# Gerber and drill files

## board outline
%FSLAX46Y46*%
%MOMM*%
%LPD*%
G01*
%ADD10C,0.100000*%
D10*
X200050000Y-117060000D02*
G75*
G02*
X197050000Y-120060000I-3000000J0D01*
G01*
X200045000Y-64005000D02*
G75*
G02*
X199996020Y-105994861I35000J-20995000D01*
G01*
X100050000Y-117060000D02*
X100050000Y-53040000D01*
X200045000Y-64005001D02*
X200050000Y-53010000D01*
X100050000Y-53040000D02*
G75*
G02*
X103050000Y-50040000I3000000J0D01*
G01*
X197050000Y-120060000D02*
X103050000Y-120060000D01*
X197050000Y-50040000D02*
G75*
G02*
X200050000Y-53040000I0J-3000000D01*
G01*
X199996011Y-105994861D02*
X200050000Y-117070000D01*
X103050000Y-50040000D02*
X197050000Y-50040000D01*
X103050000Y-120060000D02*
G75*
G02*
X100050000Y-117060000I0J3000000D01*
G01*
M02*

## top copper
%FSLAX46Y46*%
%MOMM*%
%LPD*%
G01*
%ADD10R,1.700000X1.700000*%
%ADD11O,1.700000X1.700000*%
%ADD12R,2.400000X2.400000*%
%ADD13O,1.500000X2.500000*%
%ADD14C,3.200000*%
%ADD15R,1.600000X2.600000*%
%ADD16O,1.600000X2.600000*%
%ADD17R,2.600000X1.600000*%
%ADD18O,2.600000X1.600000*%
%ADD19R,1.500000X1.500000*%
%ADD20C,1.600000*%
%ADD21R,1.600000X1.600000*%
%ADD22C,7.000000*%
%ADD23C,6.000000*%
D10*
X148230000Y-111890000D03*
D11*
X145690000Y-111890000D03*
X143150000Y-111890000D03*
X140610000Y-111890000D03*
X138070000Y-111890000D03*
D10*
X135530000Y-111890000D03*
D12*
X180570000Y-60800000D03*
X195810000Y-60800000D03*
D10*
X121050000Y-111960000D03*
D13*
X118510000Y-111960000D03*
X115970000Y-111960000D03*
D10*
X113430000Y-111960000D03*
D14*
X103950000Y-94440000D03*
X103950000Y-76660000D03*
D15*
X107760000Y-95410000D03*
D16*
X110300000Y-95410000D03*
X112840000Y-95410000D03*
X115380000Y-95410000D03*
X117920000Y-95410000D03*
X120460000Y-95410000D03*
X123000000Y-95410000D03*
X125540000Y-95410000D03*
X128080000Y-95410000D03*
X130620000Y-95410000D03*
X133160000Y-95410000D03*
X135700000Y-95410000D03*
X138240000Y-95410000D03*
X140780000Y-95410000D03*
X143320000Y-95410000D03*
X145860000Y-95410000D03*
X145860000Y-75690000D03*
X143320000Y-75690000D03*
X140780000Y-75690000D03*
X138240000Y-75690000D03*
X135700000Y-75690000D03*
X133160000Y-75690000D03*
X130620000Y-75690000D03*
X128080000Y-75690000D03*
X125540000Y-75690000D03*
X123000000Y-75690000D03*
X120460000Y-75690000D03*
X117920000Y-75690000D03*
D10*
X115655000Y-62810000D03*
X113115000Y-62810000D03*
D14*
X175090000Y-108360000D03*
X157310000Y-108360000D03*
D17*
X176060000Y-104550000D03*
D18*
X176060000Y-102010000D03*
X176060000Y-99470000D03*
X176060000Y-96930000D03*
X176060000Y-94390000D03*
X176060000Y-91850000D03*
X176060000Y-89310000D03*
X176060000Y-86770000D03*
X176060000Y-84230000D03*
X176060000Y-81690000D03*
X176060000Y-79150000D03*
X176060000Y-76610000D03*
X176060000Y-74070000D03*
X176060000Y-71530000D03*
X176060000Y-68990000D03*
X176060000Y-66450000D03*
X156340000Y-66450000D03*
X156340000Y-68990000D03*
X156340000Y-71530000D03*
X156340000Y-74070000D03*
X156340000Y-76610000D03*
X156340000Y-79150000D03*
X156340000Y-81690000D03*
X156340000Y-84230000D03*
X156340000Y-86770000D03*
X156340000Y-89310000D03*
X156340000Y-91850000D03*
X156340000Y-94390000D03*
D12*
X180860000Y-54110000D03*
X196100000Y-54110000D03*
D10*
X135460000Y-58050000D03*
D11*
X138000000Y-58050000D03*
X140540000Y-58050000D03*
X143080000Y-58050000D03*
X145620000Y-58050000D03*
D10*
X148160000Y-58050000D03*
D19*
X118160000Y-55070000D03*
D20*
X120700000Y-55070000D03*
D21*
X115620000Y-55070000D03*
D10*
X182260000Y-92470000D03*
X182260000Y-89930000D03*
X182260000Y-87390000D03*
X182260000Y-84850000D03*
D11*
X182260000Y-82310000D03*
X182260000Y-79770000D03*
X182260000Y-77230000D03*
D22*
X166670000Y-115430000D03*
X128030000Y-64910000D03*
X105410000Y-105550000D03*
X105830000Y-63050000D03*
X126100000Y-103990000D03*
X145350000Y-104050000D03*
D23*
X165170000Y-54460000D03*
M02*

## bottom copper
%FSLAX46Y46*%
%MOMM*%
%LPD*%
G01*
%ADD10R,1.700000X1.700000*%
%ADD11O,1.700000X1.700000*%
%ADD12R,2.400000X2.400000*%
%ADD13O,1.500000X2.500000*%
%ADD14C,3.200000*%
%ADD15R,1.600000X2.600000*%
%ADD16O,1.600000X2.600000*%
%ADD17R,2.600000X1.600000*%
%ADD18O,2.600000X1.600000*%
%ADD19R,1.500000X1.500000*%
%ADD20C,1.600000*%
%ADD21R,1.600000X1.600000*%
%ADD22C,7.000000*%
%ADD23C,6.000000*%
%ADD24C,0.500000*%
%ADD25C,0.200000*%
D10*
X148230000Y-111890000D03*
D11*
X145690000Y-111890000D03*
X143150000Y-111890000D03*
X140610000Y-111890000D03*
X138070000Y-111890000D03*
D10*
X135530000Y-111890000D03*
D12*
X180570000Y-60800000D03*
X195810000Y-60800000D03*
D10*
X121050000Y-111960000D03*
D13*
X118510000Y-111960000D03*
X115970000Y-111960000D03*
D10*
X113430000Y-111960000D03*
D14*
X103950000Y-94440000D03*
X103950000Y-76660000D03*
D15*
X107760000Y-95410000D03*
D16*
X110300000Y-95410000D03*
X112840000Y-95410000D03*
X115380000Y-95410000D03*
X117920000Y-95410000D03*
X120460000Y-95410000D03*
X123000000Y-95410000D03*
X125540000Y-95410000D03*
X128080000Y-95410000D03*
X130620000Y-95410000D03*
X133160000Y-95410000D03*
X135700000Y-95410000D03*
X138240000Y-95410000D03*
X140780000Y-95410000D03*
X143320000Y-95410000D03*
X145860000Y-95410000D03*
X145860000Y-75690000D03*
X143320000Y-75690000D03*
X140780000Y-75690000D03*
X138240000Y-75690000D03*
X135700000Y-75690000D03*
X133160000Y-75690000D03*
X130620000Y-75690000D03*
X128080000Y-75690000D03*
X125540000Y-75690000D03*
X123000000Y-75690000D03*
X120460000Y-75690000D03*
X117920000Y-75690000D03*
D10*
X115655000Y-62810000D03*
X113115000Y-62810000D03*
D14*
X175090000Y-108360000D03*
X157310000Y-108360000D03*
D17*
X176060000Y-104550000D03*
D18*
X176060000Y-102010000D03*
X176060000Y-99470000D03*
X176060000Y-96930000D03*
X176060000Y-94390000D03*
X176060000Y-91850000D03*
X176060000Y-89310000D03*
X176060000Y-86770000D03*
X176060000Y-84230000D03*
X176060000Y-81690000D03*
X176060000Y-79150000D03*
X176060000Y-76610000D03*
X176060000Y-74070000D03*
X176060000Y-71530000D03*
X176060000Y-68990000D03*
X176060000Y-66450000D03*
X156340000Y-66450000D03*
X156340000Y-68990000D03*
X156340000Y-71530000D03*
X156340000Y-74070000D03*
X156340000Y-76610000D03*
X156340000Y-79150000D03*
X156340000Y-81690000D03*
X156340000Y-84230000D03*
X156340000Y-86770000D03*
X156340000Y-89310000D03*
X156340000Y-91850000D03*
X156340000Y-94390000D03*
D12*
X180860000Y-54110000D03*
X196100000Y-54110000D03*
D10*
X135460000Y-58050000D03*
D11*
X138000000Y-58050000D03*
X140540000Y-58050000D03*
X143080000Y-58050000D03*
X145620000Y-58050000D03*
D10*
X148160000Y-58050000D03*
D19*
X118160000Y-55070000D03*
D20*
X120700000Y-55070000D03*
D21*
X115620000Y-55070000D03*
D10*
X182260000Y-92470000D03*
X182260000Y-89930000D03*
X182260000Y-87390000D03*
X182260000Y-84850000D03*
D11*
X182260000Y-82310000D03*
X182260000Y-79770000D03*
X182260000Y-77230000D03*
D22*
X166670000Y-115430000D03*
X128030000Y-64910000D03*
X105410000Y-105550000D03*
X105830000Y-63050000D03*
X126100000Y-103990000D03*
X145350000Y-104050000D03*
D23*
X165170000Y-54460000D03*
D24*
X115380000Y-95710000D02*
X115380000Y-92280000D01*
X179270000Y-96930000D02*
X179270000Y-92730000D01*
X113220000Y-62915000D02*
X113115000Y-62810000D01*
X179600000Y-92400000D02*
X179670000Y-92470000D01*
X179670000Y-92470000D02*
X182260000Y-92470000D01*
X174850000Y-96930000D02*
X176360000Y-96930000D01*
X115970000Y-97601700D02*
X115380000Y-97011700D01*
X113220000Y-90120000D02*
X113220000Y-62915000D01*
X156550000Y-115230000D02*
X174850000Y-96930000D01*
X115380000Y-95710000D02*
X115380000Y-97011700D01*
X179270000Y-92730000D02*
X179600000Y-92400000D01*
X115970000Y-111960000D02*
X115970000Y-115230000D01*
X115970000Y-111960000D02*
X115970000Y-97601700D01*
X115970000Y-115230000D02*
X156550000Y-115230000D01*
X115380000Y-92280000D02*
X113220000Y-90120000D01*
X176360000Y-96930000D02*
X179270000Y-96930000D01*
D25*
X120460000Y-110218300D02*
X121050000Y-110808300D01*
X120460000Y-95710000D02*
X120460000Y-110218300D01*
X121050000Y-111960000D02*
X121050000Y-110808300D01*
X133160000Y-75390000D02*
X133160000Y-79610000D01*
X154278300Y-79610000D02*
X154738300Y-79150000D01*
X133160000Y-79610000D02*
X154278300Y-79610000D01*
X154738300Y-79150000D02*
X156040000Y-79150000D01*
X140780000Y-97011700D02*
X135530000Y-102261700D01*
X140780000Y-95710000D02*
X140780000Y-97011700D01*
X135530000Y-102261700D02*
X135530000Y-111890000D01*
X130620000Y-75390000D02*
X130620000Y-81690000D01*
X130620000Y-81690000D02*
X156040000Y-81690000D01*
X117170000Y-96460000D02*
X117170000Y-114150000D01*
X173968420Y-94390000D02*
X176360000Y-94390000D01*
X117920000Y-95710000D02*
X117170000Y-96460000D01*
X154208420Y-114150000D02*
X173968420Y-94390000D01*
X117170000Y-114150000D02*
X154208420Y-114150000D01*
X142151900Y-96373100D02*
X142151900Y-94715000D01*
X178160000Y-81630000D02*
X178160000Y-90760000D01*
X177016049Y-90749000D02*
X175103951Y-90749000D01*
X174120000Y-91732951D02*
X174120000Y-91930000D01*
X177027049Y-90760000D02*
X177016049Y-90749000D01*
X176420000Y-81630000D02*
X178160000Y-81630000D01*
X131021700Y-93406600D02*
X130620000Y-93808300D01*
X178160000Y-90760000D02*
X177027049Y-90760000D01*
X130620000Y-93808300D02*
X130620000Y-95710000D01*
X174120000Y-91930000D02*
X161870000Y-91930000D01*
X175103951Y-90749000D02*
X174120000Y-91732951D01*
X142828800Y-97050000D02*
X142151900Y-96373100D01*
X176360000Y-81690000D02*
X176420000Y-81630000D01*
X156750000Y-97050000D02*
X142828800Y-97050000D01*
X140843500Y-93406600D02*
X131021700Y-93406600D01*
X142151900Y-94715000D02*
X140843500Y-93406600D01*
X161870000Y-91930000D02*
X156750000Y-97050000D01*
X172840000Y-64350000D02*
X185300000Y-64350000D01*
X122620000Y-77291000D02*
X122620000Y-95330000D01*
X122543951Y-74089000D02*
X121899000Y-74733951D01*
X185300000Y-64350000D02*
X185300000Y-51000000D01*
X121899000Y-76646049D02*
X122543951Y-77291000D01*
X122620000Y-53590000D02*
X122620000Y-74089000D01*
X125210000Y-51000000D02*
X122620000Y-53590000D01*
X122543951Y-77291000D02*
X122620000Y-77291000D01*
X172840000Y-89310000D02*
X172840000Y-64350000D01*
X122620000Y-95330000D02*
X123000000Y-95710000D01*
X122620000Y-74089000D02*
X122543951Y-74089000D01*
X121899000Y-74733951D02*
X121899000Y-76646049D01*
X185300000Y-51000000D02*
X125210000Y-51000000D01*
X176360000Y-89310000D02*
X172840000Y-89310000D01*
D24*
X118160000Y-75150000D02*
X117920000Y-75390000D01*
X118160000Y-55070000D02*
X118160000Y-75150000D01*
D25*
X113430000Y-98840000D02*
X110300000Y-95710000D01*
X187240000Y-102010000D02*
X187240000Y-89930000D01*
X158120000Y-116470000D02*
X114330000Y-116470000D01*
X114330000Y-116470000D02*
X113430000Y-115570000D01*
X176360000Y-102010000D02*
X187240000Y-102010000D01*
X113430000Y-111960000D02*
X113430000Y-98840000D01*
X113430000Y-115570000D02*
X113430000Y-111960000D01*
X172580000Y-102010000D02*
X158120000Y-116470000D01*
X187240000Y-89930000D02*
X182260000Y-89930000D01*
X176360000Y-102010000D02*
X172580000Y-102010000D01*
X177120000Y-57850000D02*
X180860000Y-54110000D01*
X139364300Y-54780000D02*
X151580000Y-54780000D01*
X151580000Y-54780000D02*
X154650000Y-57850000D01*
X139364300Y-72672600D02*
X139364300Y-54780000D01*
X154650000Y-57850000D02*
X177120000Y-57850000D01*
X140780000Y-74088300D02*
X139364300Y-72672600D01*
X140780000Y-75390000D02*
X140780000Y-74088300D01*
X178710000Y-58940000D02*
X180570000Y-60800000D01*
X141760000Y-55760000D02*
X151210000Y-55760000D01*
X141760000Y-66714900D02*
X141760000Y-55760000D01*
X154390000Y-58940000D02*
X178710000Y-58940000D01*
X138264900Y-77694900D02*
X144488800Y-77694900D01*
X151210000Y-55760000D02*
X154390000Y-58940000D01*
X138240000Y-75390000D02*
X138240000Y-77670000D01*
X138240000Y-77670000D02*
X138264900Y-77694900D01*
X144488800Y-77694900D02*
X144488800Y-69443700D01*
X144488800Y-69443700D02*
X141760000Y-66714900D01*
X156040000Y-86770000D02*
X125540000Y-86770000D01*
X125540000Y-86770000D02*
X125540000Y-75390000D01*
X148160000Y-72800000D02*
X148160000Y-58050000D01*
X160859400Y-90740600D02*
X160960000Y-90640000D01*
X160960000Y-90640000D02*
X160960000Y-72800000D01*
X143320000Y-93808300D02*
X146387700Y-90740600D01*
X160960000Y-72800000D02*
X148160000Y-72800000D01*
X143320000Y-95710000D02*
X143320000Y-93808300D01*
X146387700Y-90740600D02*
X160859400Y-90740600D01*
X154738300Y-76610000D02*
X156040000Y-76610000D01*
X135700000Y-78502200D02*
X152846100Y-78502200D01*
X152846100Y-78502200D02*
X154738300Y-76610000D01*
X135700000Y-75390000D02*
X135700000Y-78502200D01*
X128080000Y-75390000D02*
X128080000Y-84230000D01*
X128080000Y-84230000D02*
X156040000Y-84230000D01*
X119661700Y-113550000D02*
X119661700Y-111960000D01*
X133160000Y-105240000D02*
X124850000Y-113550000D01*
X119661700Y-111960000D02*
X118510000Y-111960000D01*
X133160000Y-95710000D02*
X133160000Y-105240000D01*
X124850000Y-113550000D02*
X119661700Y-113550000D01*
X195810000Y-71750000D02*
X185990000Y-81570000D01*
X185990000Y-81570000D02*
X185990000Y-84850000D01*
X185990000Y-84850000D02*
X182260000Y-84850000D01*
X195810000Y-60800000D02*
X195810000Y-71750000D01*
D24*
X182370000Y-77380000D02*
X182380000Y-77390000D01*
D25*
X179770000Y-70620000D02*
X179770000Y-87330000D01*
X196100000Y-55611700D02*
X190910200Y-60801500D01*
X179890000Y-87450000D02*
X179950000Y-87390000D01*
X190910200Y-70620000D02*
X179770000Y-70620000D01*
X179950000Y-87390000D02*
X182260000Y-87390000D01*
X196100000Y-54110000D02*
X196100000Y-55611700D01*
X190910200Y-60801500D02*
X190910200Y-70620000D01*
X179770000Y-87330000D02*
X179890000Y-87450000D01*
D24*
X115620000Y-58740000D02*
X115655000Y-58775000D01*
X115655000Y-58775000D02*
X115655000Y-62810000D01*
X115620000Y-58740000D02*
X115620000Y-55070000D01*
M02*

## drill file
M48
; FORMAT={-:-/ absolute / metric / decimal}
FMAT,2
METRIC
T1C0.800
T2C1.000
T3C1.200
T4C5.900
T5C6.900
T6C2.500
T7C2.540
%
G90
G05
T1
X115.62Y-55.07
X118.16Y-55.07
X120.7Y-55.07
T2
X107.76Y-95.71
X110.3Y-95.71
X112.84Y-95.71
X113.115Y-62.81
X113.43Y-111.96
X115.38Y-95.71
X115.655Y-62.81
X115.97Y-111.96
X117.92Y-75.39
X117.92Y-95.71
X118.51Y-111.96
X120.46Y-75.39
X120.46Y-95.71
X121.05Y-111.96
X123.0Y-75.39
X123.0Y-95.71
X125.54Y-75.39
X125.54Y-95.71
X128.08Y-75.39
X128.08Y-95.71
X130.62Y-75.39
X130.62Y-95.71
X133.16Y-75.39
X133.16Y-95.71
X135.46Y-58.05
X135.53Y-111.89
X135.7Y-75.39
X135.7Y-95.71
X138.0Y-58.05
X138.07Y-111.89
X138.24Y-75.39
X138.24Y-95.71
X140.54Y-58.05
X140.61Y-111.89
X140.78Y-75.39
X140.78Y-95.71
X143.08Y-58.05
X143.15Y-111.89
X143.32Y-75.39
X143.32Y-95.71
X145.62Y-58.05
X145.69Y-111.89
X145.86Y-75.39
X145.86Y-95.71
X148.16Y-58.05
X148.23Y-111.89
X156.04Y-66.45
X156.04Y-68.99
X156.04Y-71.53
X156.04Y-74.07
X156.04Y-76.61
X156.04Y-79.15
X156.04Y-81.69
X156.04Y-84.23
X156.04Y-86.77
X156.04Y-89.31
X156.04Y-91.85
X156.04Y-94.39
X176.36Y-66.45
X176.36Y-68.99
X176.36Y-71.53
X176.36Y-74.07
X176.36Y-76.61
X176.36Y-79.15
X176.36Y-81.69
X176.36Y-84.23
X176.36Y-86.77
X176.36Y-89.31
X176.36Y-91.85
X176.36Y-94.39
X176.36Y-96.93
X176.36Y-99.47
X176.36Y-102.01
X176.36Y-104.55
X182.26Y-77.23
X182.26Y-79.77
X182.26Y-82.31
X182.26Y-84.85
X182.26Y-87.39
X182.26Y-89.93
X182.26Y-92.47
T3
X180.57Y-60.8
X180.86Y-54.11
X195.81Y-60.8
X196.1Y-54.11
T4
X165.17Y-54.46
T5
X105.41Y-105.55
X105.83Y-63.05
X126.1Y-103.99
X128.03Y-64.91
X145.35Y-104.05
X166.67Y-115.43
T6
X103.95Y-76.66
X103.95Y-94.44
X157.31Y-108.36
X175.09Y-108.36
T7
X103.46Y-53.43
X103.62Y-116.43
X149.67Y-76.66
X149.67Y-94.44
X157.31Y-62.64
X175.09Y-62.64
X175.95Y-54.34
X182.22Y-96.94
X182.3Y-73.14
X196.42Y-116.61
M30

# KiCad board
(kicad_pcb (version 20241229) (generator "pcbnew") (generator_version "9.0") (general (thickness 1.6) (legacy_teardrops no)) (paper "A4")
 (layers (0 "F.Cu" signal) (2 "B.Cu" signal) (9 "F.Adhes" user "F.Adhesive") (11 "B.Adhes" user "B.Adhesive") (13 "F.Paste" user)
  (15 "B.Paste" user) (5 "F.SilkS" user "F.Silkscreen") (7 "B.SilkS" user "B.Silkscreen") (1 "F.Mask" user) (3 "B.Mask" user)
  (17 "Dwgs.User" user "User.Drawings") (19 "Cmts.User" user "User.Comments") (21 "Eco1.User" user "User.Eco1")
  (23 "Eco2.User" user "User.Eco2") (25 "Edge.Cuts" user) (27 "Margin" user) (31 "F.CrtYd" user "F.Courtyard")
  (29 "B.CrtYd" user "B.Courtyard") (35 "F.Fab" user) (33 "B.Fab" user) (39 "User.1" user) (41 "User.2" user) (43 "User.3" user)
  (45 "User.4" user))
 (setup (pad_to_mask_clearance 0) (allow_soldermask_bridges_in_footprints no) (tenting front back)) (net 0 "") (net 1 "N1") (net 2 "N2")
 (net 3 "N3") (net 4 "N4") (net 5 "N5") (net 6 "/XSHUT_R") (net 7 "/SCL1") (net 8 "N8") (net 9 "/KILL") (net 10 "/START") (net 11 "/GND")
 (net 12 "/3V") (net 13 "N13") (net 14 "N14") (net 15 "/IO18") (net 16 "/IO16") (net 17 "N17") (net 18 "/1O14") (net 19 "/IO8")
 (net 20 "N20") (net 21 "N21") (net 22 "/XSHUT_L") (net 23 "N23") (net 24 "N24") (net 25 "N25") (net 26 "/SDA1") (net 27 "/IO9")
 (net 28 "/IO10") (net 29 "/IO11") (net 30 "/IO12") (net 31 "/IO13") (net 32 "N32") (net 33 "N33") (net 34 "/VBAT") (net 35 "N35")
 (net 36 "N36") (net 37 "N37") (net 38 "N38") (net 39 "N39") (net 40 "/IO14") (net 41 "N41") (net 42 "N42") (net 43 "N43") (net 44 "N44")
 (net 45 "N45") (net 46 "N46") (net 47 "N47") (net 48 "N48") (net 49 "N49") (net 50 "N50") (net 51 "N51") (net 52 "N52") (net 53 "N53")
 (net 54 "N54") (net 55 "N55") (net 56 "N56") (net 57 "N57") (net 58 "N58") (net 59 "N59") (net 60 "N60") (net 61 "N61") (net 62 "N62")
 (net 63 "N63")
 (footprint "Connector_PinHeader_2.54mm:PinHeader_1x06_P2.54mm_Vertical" (layer "F.Cu") (at 148.23 111.89 -90)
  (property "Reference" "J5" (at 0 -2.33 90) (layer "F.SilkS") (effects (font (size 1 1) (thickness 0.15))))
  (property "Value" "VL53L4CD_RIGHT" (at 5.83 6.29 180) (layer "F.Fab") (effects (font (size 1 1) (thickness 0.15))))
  (pad "1" thru_hole rect (at 0 0 270) (size 1.7 1.7) (drill 1) (layers "*.Cu" "*.Mask") (remove_unused_layers no) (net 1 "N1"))
  (pad "2" thru_hole oval (at 0 2.54 270) (size 1.7 1.7) (drill 1) (layers "*.Cu" "*.Mask") (remove_unused_layers no) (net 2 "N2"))
  (pad "3" thru_hole oval (at 0 5.08 270) (size 1.7 1.7) (drill 1) (layers "*.Cu" "*.Mask") (remove_unused_layers no) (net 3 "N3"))
  (pad "4" thru_hole oval (at 0 7.62 270) (size 1.7 1.7) (drill 1) (layers "*.Cu" "*.Mask") (remove_unused_layers no) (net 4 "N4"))
  (pad "5" thru_hole oval (at 0 10.16 270) (size 1.7 1.7) (drill 1) (layers "*.Cu" "*.Mask") (remove_unused_layers no) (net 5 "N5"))
  (pad "6" thru_hole rect (at 0 12.7 270) (size 1.7 1.7) (drill 1) (layers "*.Cu" "*.Mask") (remove_unused_layers no) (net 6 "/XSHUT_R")))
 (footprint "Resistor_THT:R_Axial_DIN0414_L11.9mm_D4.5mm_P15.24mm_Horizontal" (layer "F.Cu") (at 180.57 60.8)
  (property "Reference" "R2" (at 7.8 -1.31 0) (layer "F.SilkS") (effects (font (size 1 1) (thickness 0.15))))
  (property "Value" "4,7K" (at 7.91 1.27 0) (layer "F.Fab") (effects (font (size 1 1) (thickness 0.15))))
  (pad "1" thru_hole rect (at 0 0) (size 2.4 2.4) (drill 1.2) (layers "*.Cu" "*.Mask") (remove_unused_layers no) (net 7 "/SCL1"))
  (pad "2" thru_hole rect (at 15.24 0) (size 2.4 2.4) (drill 1.2) (layers "*.Cu" "*.Mask") (remove_unused_layers no) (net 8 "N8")))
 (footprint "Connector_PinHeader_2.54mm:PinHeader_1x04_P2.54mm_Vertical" (layer "F.Cu") (at 121.05 111.96 -90)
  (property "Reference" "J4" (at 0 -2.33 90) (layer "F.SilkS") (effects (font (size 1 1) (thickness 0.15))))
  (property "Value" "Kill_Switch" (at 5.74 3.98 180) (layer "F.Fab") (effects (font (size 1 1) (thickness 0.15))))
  (pad "1" thru_hole rect (at 0 0 270) (size 1.7 1.7) (drill 1) (layers "*.Cu" "*.Mask") (remove_unused_layers no) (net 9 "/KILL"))
  (pad "2" thru_hole oval (at 0 2.54 270) (size 2.5 1.5) (drill 1) (layers "*.Cu" "*.Mask") (remove_unused_layers no) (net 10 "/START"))
  (pad "3" thru_hole oval (at 0 5.08 270) (size 2.5 1.5) (drill 1) (layers "*.Cu" "*.Mask") (remove_unused_layers no) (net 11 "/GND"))
  (pad "4" thru_hole rect (at 0 7.62 270) (size 1.7 1.7) (drill 1) (layers "*.Cu" "*.Mask") (remove_unused_layers no) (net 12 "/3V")))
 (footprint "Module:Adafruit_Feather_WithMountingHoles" (layer "F.Cu") (at 107.76 95.71 90)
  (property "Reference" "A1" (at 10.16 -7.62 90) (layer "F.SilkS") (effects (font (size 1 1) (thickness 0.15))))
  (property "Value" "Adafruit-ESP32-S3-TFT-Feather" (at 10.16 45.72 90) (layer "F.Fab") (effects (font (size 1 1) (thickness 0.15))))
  (pad "" np_thru_hole circle (at 1.27 -3.81) (size 3.2 3.2) (drill 2.5) (layers "*.Cu" "*.Mask"))
  (pad "" np_thru_hole circle (at 1.27 41.91) (size 2.54 2.54) (drill 2.54) (layers "*.Cu" "*.Mask"))
  (pad "" np_thru_hole circle (at 19.05 -3.81) (size 3.2 3.2) (drill 2.5) (layers "*.Cu" "*.Mask"))
  (pad "" np_thru_hole circle (at 19.05 41.91) (size 2.54 2.54) (drill 2.54) (layers "*.Cu" "*.Mask"))
  (pad "1" thru_hole rect (at 0 0 90) (size 2.6 1.6) (drill 1 (offset 0.3 0)) (layers "*.Cu" "*.Mask") (remove_unused_layers no)
   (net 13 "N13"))
  (pad "2" thru_hole oval (at 0 2.54 90) (size 2.6 1.6) (drill 1 (offset 0.3 0)) (layers "*.Cu" "*.Mask") (remove_unused_layers no)
   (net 12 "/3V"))
  (pad "3" thru_hole oval (at 0 5.08 90) (size 2.6 1.6) (drill 1 (offset 0.3 0)) (layers "*.Cu" "*.Mask") (remove_unused_layers no)
   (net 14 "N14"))
  (pad "4" thru_hole oval (at 0 7.62 90) (size 2.6 1.6) (drill 1 (offset 0.3 0)) (layers "*.Cu" "*.Mask") (remove_unused_layers no)
   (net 11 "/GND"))
  (pad "5" thru_hole oval (at 0 10.16 90) (size 2.6 1.6) (drill 1 (offset 0.3 0)) (layers "*.Cu" "*.Mask") (remove_unused_layers no)
   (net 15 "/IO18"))
  (pad "6" thru_hole oval (at 0 12.7 90) (size 2.6 1.6) (drill 1 (offset 0.3 0)) (layers "*.Cu" "*.Mask") (remove_unused_layers no)
   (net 9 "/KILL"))
  (pad "7" thru_hole oval (at 0 15.24 90) (size 2.6 1.6) (drill 1 (offset 0.3 0)) (layers "*.Cu" "*.Mask") (remove_unused_layers no)
   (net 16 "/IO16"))
  (pad "8" thru_hole oval (at 0 17.78 90) (size 2.6 1.6) (drill 1 (offset 0.3 0)) (layers "*.Cu" "*.Mask") (remove_unused_layers no)
   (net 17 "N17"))
  (pad "9" thru_hole oval (at 0 20.32 90) (size 2.6 1.6) (drill 1 (offset 0.3 0)) (layers "*.Cu" "*.Mask") (remove_unused_layers no)
   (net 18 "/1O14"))
  (pad "10" thru_hole oval (at 0 22.86 90) (size 2.6 1.6) (drill 1 (offset 0.3 0)) (layers "*.Cu" "*.Mask") (remove_unused_layers no)
   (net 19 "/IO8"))
  (pad "11" thru_hole oval (at 0 25.4 90) (size 2.6 1.6) (drill 1 (offset 0.3 0)) (layers "*.Cu" "*.Mask") (remove_unused_layers no)
   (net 10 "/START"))
  (pad "12" thru_hole oval (at 0 27.94 90) (size 2.6 1.6) (drill 1 (offset 0.3 0)) (layers "*.Cu" "*.Mask") (remove_unused_layers no)
   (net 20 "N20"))
  (pad "13" thru_hole oval (at 0 30.48 90) (size 2.6 1.6) (drill 1 (offset 0.3 0)) (layers "*.Cu" "*.Mask") (remove_unused_layers no)
   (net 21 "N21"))
  (pad "14" thru_hole oval (at 0 33.02 90) (size 2.6 1.6) (drill 1 (offset 0.3 0)) (layers "*.Cu" "*.Mask") (remove_unused_layers no)
   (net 6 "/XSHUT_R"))
  (pad "15" thru_hole oval (at 0 35.56 90) (size 2.6 1.6) (drill 1 (offset 0.3 0)) (layers "*.Cu" "*.Mask") (remove_unused_layers no)
   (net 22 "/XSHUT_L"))
  (pad "16" thru_hole oval (at 0 38.1 90) (size 2.6 1.6) (drill 1 (offset 0.3 0)) (layers "*.Cu" "*.Mask") (remove_unused_layers no)
   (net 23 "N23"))
  (pad "17" thru_hole oval (at 20.32 38.1 270) (size 2.6 1.6) (drill 1 (offset 0.3 0)) (layers "*.Cu" "*.Mask") (remove_unused_layers no)
   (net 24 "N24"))
  (pad "18" thru_hole oval (at 20.32 35.56 270) (size 2.6 1.6) (drill 1 (offset 0.3 0)) (layers "*.Cu" "*.Mask") (remove_unused_layers no)
   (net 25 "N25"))
  (pad "19" thru_hole oval (at 20.32 33.02 270) (size 2.6 1.6) (drill 1 (offset 0.3 0)) (layers "*.Cu" "*.Mask") (remove_unused_layers no)
   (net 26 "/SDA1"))
  (pad "20" thru_hole oval (at 20.32 30.48 270) (size 2.6 1.6) (drill 1 (offset 0.3 0)) (layers "*.Cu" "*.Mask") (remove_unused_layers no)
   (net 7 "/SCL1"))
  (pad "21" thru_hole oval (at 20.32 27.94 270) (size 2.6 1.6) (drill 1 (offset 0.3 0)) (layers "*.Cu" "*.Mask") (remove_unused_layers no)
   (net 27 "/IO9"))
  (pad "22" thru_hole oval (at 20.32 25.4 270) (size 2.6 1.6) (drill 1 (offset 0.3 0)) (layers "*.Cu" "*.Mask") (remove_unused_layers no)
   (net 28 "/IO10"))
  (pad "23" thru_hole oval (at 20.32 22.86 270) (size 2.6 1.6) (drill 1 (offset 0.3 0)) (layers "*.Cu" "*.Mask") (remove_unused_layers no)
   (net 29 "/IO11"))
  (pad "24" thru_hole oval (at 20.32 20.32 270) (size 2.6 1.6) (drill 1 (offset 0.3 0)) (layers "*.Cu" "*.Mask") (remove_unused_layers no)
   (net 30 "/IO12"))
  (pad "25" thru_hole oval (at 20.32 17.78 270) (size 2.6 1.6) (drill 1 (offset 0.3 0)) (layers "*.Cu" "*.Mask") (remove_unused_layers no)
   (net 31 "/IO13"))
  (pad "26" thru_hole oval (at 20.32 15.24 270) (size 2.6 1.6) (drill 1 (offset 0.3 0)) (layers "*.Cu" "*.Mask") (remove_unused_layers no)
   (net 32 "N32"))
  (pad "27" thru_hole oval (at 20.32 12.7 270) (size 2.6 1.6) (drill 1 (offset 0.3 0)) (layers "*.Cu" "*.Mask") (remove_unused_layers no)
   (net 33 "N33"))
  (pad "28" thru_hole oval (at 20.32 10.16 270) (size 2.6 1.6) (drill 1 (offset 0.3 0)) (layers "*.Cu" "*.Mask") (remove_unused_layers no)
   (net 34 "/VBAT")))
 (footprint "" (layer "F.Cu") (at 103.62 116.43)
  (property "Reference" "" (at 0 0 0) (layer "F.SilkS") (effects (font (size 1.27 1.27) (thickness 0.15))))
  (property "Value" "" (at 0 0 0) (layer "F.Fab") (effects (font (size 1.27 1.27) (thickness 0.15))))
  (pad "" np_thru_hole circle (at 0 0 90) (size 2.54 2.54) (drill 2.54) (layers "*.Cu" "*.Mask")))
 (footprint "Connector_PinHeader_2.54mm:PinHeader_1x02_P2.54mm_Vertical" (layer "F.Cu") (at 115.655 62.81 -90)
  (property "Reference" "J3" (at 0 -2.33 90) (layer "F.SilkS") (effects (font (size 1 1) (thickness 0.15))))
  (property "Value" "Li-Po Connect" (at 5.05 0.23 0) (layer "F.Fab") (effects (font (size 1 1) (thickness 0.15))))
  (pad "1" thru_hole rect (at 0 0 270) (size 1.7 1.7) (drill 1) (layers "*.Cu" "*.Mask") (remove_unused_layers no) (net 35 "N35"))
  (pad "2" thru_hole rect (at 0 2.54 270) (size 1.7 1.7) (drill 1) (layers "*.Cu" "*.Mask") (remove_unused_layers no) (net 11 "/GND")))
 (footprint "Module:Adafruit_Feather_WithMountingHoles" (layer "F.Cu") (at 176.36 104.55 180)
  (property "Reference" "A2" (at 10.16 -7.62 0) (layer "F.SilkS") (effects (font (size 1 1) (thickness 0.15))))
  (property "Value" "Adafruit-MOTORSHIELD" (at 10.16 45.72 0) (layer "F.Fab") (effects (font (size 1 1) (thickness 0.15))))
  (pad "" np_thru_hole circle (at 1.27 -3.81 90) (size 3.2 3.2) (drill 2.5) (layers "*.Cu" "*.Mask"))
  (pad "" np_thru_hole circle (at 1.27 41.91 90) (size 2.54 2.54) (drill 2.54) (layers "*.Cu" "*.Mask"))
  (pad "" np_thru_hole circle (at 19.05 -3.81 90) (size 3.2 3.2) (drill 2.5) (layers "*.Cu" "*.Mask"))
  (pad "" np_thru_hole circle (at 19.05 41.91 90) (size 2.54 2.54) (drill 2.54) (layers "*.Cu" "*.Mask"))
  (pad "1" thru_hole rect (at 0 0 180) (size 2.6 1.6) (drill 1 (offset 0.3 0)) (layers "*.Cu" "*.Mask") (remove_unused_layers no)
   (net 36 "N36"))
  (pad "2" thru_hole oval (at 0 2.54 180) (size 2.6 1.6) (drill 1 (offset 0.3 0)) (layers "*.Cu" "*.Mask") (remove_unused_layers no)
   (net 12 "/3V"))
  (pad "3" thru_hole oval (at 0 5.08 180) (size 2.6 1.6) (drill 1 (offset 0.3 0)) (layers "*.Cu" "*.Mask") (remove_unused_layers no)
   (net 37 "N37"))
  (pad "4" thru_hole oval (at 0 7.62 180) (size 2.6 1.6) (drill 1 (offset 0.3 0)) (layers "*.Cu" "*.Mask") (remove_unused_layers no)
   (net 11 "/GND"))
  (pad "5" thru_hole oval (at 0 10.16 180) (size 2.6 1.6) (drill 1 (offset 0.3 0)) (layers "*.Cu" "*.Mask") (remove_unused_layers no)
   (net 15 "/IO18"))
  (pad "6" thru_hole oval (at 0 12.7 180) (size 2.6 1.6) (drill 1 (offset 0.3 0)) (layers "*.Cu" "*.Mask") (remove_unused_layers no)
   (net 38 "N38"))
  (pad "7" thru_hole oval (at 0 15.24 180) (size 2.6 1.6) (drill 1 (offset 0.3 0)) (layers "*.Cu" "*.Mask") (remove_unused_layers no)
   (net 16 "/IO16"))
  (pad "8" thru_hole oval (at 0 17.78 180) (size 2.6 1.6) (drill 1 (offset 0.3 0)) (layers "*.Cu" "*.Mask") (remove_unused_layers no)
   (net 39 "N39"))
  (pad "9" thru_hole oval (at 0 20.32 180) (size 2.6 1.6) (drill 1 (offset 0.3 0)) (layers "*.Cu" "*.Mask") (remove_unused_layers no)
   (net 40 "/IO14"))
  (pad "10" thru_hole oval (at 0 22.86 180) (size 2.6 1.6) (drill 1 (offset 0.3 0)) (layers "*.Cu" "*.Mask") (remove_unused_layers no)
   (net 19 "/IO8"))
  (pad "11" thru_hole oval (at 0 25.4 180) (size 2.6 1.6) (drill 1 (offset 0.3 0)) (layers "*.Cu" "*.Mask") (remove_unused_layers no)
   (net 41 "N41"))
  (pad "12" thru_hole oval (at 0 27.94 180) (size 2.6 1.6) (drill 1 (offset 0.3 0)) (layers "*.Cu" "*.Mask") (remove_unused_layers no)
   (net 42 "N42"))
  (pad "13" thru_hole oval (at 0 30.48 180) (size 2.6 1.6) (drill 1 (offset 0.3 0)) (layers "*.Cu" "*.Mask") (remove_unused_layers no)
   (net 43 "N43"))
  (pad "14" thru_hole oval (at 0 33.02 180) (size 2.6 1.6) (drill 1 (offset 0.3 0)) (layers "*.Cu" "*.Mask") (remove_unused_layers no)
   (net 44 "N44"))
  (pad "15" thru_hole oval (at 0 35.56 180) (size 2.6 1.6) (drill 1 (offset 0.3 0)) (layers "*.Cu" "*.Mask") (remove_unused_layers no)
   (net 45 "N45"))
  (pad "16" thru_hole oval (at 0 38.1 180) (size 2.6 1.6) (drill 1 (offset 0.3 0)) (layers "*.Cu" "*.Mask") (remove_unused_layers no)
   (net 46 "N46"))
  (pad "17" thru_hole oval (at 20.32 38.1) (size 2.6 1.6) (drill 1 (offset 0.3 0)) (layers "*.Cu" "*.Mask") (remove_unused_layers no)
   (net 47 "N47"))
  (pad "18" thru_hole oval (at 20.32 35.56) (size 2.6 1.6) (drill 1 (offset 0.3 0)) (layers "*.Cu" "*.Mask") (remove_unused_layers no)
   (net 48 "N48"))
  (pad "19" thru_hole oval (at 20.32 33.02) (size 2.6 1.6) (drill 1 (offset 0.3 0)) (layers "*.Cu" "*.Mask") (remove_unused_layers no)
   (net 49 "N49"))
  (pad "20" thru_hole oval (at 20.32 30.48) (size 2.6 1.6) (drill 1 (offset 0.3 0)) (layers "*.Cu" "*.Mask") (remove_unused_layers no)
   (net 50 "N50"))
  (pad "21" thru_hole oval (at 20.32 27.94) (size 2.6 1.6) (drill 1 (offset 0.3 0)) (layers "*.Cu" "*.Mask") (remove_unused_layers no)
   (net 27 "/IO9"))
  (pad "22" thru_hole oval (at 20.32 25.4) (size 2.6 1.6) (drill 1 (offset 0.3 0)) (layers "*.Cu" "*.Mask") (remove_unused_layers no)
   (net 28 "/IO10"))
  (pad "23" thru_hole oval (at 20.32 22.86) (size 2.6 1.6) (drill 1 (offset 0.3 0)) (layers "*.Cu" "*.Mask") (remove_unused_layers no)
   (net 29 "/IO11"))
  (pad "24" thru_hole oval (at 20.32 20.32) (size 2.6 1.6) (drill 1 (offset 0.3 0)) (layers "*.Cu" "*.Mask") (remove_unused_layers no)
   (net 30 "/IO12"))
  (pad "25" thru_hole oval (at 20.32 17.78) (size 2.6 1.6) (drill 1 (offset 0.3 0)) (layers "*.Cu" "*.Mask") (remove_unused_layers no)
   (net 31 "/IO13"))
  (pad "26" thru_hole oval (at 20.32 15.24) (size 2.6 1.6) (drill 1 (offset 0.3 0)) (layers "*.Cu" "*.Mask") (remove_unused_layers no)
   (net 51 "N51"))
  (pad "27" thru_hole oval (at 20.32 12.7) (size 2.6 1.6) (drill 1 (offset 0.3 0)) (layers "*.Cu" "*.Mask") (remove_unused_layers no)
   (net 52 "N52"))
  (pad "28" thru_hole oval (at 20.32 10.16) (size 2.6 1.6) (drill 1 (offset 0.3 0)) (layers "*.Cu" "*.Mask") (remove_unused_layers no)
   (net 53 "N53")))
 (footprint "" (layer "F.Cu") (at 182.3 73.14)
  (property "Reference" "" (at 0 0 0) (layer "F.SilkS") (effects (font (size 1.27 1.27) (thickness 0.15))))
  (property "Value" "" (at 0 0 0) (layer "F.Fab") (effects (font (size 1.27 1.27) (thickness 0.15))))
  (pad "" np_thru_hole circle (at 0 0 90) (size 2.54 2.54) (drill 2.54) (layers "*.Cu" "*.Mask")))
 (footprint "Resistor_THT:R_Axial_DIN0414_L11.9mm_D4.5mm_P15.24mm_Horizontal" (layer "F.Cu") (at 180.86 54.11)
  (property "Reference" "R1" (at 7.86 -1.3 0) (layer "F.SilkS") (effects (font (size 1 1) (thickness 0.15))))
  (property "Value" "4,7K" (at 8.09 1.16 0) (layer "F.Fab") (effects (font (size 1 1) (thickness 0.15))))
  (pad "1" thru_hole rect (at 0 0) (size 2.4 2.4) (drill 1.2) (layers "*.Cu" "*.Mask") (remove_unused_layers no) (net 26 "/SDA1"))
  (pad "2" thru_hole rect (at 15.24 0) (size 2.4 2.4) (drill 1.2) (layers "*.Cu" "*.Mask") (remove_unused_layers no) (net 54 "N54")))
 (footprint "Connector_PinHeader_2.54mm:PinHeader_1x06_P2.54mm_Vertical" (layer "F.Cu") (at 135.46 58.05 90)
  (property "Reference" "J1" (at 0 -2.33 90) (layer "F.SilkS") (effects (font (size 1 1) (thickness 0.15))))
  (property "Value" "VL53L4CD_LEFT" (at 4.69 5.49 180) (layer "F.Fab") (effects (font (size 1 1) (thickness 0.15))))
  (pad "1" thru_hole rect (at 0 0 90) (size 1.7 1.7) (drill 1) (layers "*.Cu" "*.Mask") (remove_unused_layers no) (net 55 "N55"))
  (pad "2" thru_hole oval (at 0 2.54 90) (size 1.7 1.7) (drill 1) (layers "*.Cu" "*.Mask") (remove_unused_layers no) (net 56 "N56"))
  (pad "3" thru_hole oval (at 0 5.08 90) (size 1.7 1.7) (drill 1) (layers "*.Cu" "*.Mask") (remove_unused_layers no) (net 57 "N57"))
  (pad "4" thru_hole oval (at 0 7.62 90) (size 1.7 1.7) (drill 1) (layers "*.Cu" "*.Mask") (remove_unused_layers no) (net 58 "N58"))
  (pad "5" thru_hole oval (at 0 10.16 90) (size 1.7 1.7) (drill 1) (layers "*.Cu" "*.Mask") (remove_unused_layers no) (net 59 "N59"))
  (pad "6" thru_hole rect (at 0 12.7 90) (size 1.7 1.7) (drill 1) (layers "*.Cu" "*.Mask") (remove_unused_layers no) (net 22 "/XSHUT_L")))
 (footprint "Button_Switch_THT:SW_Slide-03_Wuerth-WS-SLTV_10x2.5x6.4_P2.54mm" (layer "F.Cu") (at 118.16 55.07 180)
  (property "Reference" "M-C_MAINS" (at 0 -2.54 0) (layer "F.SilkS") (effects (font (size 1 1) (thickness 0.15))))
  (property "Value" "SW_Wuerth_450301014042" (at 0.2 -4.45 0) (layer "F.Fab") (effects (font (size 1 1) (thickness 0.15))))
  (pad "1" thru_hole rect (at 0 0 180) (size 1.5 1.5) (drill 0.8) (layers "*.Cu" "*.Mask") (remove_unused_layers no) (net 34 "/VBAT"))
  (pad "2" thru_hole circle (at -2.54 0 180) (size 1.6 1.6) (drill 0.8) (layers "*.Cu" "*.Mask") (remove_unused_layers no) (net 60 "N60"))
  (pad "3" thru_hole rect (at 2.54 0 180) (size 1.6 1.6) (drill 0.8) (layers "*.Cu" "*.Mask") (remove_unused_layers no) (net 35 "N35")))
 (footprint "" (layer "F.Cu") (at 182.22 96.94)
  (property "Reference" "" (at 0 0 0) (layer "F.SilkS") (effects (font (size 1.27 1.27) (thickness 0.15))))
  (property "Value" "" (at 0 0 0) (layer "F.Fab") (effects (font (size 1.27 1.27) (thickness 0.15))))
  (pad "" np_thru_hole circle (at 0 0 90) (size 2.54 2.54) (drill 2.54) (layers "*.Cu" "*.Mask")))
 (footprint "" (layer "F.Cu") (at 196.42 116.61)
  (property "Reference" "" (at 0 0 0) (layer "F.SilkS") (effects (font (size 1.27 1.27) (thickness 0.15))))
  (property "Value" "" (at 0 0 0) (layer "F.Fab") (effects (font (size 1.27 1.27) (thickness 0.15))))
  (pad "" np_thru_hole circle (at 0 0 90) (size 2.54 2.54) (drill 2.54) (layers "*.Cu" "*.Mask")))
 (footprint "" (layer "F.Cu") (at 175.95 54.34)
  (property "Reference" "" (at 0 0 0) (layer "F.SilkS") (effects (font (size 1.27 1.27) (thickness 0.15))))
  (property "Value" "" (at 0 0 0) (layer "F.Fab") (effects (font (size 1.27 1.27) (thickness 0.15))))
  (pad "" np_thru_hole circle (at 0 0 90) (size 2.54 2.54) (drill 2.54) (layers "*.Cu" "*.Mask")))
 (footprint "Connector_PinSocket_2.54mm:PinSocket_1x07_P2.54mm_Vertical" (layer "F.Cu") (at 182.26 92.47 180)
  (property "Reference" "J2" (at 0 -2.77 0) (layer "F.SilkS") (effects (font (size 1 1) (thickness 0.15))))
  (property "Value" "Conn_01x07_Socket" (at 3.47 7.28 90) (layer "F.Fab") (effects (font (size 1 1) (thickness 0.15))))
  (pad "1" thru_hole rect (at 0 0 180) (size 1.7 1.7) (drill 1) (layers "*.Cu" "*.Mask") (remove_unused_layers no) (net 11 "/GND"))
  (pad "2" thru_hole rect (at 0 2.54 180) (size 1.7 1.7) (drill 1) (layers "*.Cu" "*.Mask") (remove_unused_layers no) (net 12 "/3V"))
  (pad "3" thru_hole rect (at 0 5.08 180) (size 1.7 1.7) (drill 1) (layers "*.Cu" "*.Mask") (remove_unused_layers no) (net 54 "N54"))
  (pad "4" thru_hole rect (at 0 7.62 180) (size 1.7 1.7) (drill 1) (layers "*.Cu" "*.Mask") (remove_unused_layers no) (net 8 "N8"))
  (pad "5" thru_hole oval (at 0 10.16 180) (size 1.7 1.7) (drill 1) (layers "*.Cu" "*.Mask") (remove_unused_layers no) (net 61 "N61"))
  (pad "6" thru_hole oval (at 0 12.7 180) (size 1.7 1.7) (drill 1) (layers "*.Cu" "*.Mask") (remove_unused_layers no) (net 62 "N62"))
  (pad "7" thru_hole oval (at 0 15.24 180) (size 1.7 1.7) (drill 1) (layers "*.Cu" "*.Mask") (remove_unused_layers no) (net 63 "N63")))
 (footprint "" (layer "F.Cu") (at 103.46 53.43)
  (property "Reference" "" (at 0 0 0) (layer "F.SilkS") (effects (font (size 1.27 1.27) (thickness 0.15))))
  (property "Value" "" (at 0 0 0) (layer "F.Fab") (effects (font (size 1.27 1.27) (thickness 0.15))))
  (pad "" np_thru_hole circle (at 0 0 90) (size 2.54 2.54) (drill 2.54) (layers "*.Cu" "*.Mask")))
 (gr_arc (start 200.05 117.06) (mid 199.17132 119.18132) (end 197.05 120.06) (stroke (width 0.1) (type default)) (layer "Edge.Cuts"))
 (gr_arc (start 200.045 64.005) (mid 221.075015 85.02449) (end 199.99602 105.994861) (stroke (width 0.1) (type solid)) (layer "Edge.Cuts"))
 (gr_line (start 100.05 117.06) (end 100.05 53.04) (stroke (width 0.1) (type default)) (layer "Edge.Cuts"))
 (gr_line (start 200.045 64.005001) (end 200.05 53.01) (stroke (width 0.1) (type solid)) (layer "Edge.Cuts"))
 (gr_arc (start 100.05 53.04) (mid 100.92868 50.91868) (end 103.05 50.04) (stroke (width 0.1) (type default)) (layer "Edge.Cuts"))
 (gr_line (start 197.05 120.06) (end 103.05 120.06) (stroke (width 0.1) (type default)) (layer "Edge.Cuts"))
 (gr_arc (start 197.05 50.04) (mid 199.17132 50.91868) (end 200.05 53.04) (stroke (width 0.1) (type default)) (layer "Edge.Cuts"))
 (gr_line (start 199.996011 105.994861) (end 200.05 117.07) (stroke (width 0.1) (type solid)) (layer "Edge.Cuts"))
 (gr_line (start 103.05 50.04) (end 197.05 50.04) (stroke (width 0.1) (type default)) (layer "Edge.Cuts"))
 (gr_arc (start 103.05 120.06) (mid 100.92868 119.18132) (end 100.05 117.06) (stroke (width 0.1) (type default)) (layer "Edge.Cuts"))
 (via (at 166.67 115.43) (size 7) (drill 6.9) (layers "F.Cu" "B.Cu") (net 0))
 (via (at 128.03 64.91) (size 7) (drill 6.9) (layers "F.Cu" "B.Cu") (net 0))
 (via (at 105.41 105.55) (size 7) (drill 6.9) (layers "F.Cu" "B.Cu") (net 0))
 (via (at 105.83 63.05) (size 7) (drill 6.9) (layers "F.Cu" "B.Cu") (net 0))
 (via (at 126.1 103.99) (size 7) (drill 6.9) (layers "F.Cu" "B.Cu") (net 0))
 (via (at 145.35 104.05) (size 7) (drill 6.9) (layers "F.Cu" "B.Cu") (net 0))
 (via (at 165.17 54.46) (size 6) (drill 5.9) (layers "F.Cu" "B.Cu") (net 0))
 (segment (start 115.38 95.71) (end 115.38 92.28) (width 0.5) (layer "B.Cu") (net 11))
 (segment (start 179.27 96.93) (end 179.27 92.73) (width 0.5) (layer "B.Cu") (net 11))
 (segment (start 113.22 62.915) (end 113.115 62.81) (width 0.5) (layer "B.Cu") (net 11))
 (segment (start 179.6 92.4) (end 179.67 92.47) (width 0.5) (layer "B.Cu") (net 11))
 (segment (start 179.67 92.47) (end 182.26 92.47) (width 0.5) (layer "B.Cu") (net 11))
 (segment (start 174.85 96.93) (end 176.36 96.93) (width 0.5) (layer "B.Cu") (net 11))
 (segment (start 115.97 97.6017) (end 115.38 97.0117) (width 0.5) (layer "B.Cu") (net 11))
 (segment (start 113.22 90.12) (end 113.22 62.915) (width 0.5) (layer "B.Cu") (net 11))
 (segment (start 156.55 115.23) (end 174.85 96.93) (width 0.5) (layer "B.Cu") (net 11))
 (segment (start 115.38 95.71) (end 115.38 97.0117) (width 0.5) (layer "B.Cu") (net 11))
 (segment (start 179.27 92.73) (end 179.6 92.4) (width 0.5) (layer "B.Cu") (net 11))
 (segment (start 115.97 111.96) (end 115.97 115.23) (width 0.5) (layer "B.Cu") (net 11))
 (segment (start 115.97 111.96) (end 115.97 97.6017) (width 0.5) (layer "B.Cu") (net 11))
 (segment (start 115.97 115.23) (end 156.55 115.23) (width 0.5) (layer "B.Cu") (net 11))
 (segment (start 115.38 92.28) (end 113.22 90.12) (width 0.5) (layer "B.Cu") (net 11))
 (segment (start 176.36 96.93) (end 179.27 96.93) (width 0.5) (layer "B.Cu") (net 11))
 (segment (start 120.46 110.2183) (end 121.05 110.8083) (width 0.2) (layer "B.Cu") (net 9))
 (segment (start 120.46 95.71) (end 120.46 110.2183) (width 0.2) (layer "B.Cu") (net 9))
 (segment (start 121.05 111.96) (end 121.05 110.8083) (width 0.2) (layer "B.Cu") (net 9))
 (segment (start 133.16 75.39) (end 133.16 79.61) (width 0.2) (layer "B.Cu") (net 28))
 (segment (start 154.2783 79.61) (end 154.7383 79.15) (width 0.2) (layer "B.Cu") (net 28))
 (segment (start 133.16 79.61) (end 154.2783 79.61) (width 0.2) (layer "B.Cu") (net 28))
 (segment (start 154.7383 79.15) (end 156.04 79.15) (width 0.2) (layer "B.Cu") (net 28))
 (segment (start 140.78 97.0117) (end 135.53 102.2617) (width 0.2) (layer "B.Cu") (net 6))
 (segment (start 140.78 95.71) (end 140.78 97.0117) (width 0.2) (layer "B.Cu") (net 6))
 (segment (start 135.53 102.2617) (end 135.53 111.89) (width 0.2) (layer "B.Cu") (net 6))
 (segment (start 130.62 75.39) (end 130.62 81.69) (width 0.2) (layer "B.Cu") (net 29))
 (segment (start 130.62 81.69) (end 156.04 81.69) (width 0.2) (layer "B.Cu") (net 29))
 (segment (start 117.17 96.46) (end 117.17 114.15) (width 0.2) (layer "B.Cu") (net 15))
 (segment (start 173.96842 94.39) (end 176.36 94.39) (width 0.2) (layer "B.Cu") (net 15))
 (segment (start 117.92 95.71) (end 117.17 96.46) (width 0.2) (layer "B.Cu") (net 15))
 (segment (start 154.20842 114.15) (end 173.96842 94.39) (width 0.2) (layer "B.Cu") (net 15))
 (segment (start 117.17 114.15) (end 154.20842 114.15) (width 0.2) (layer "B.Cu") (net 15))
 (segment (start 142.1519 96.3731) (end 142.1519 94.715) (width 0.2) (layer "B.Cu") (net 19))
 (segment (start 178.16 81.63) (end 178.16 90.76) (width 0.2) (layer "B.Cu") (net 19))
 (segment (start 177.016049 90.749) (end 175.103951 90.749) (width 0.2) (layer "B.Cu") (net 19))
 (segment (start 174.12 91.732951) (end 174.12 91.93) (width 0.2) (layer "B.Cu") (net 19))
 (segment (start 177.027049 90.76) (end 177.016049 90.749) (width 0.2) (layer "B.Cu") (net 19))
 (segment (start 176.42 81.63) (end 178.16 81.63) (width 0.2) (layer "B.Cu") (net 19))
 (segment (start 131.0217 93.4066) (end 130.62 93.8083) (width 0.2) (layer "B.Cu") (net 19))
 (segment (start 178.16 90.76) (end 177.027049 90.76) (width 0.2) (layer "B.Cu") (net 19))
 (segment (start 130.62 93.8083) (end 130.62 95.71) (width 0.2) (layer "B.Cu") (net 19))
 (segment (start 174.12 91.93) (end 161.87 91.93) (width 0.2) (layer "B.Cu") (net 19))
 (segment (start 175.103951 90.749) (end 174.12 91.732951) (width 0.2) (layer "B.Cu") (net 19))
 (segment (start 142.8288 97.05) (end 142.1519 96.3731) (width 0.2) (layer "B.Cu") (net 19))
 (segment (start 176.36 81.69) (end 176.42 81.63) (width 0.2) (layer "B.Cu") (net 19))
 (segment (start 156.75 97.05) (end 142.8288 97.05) (width 0.2) (layer "B.Cu") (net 19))
 (segment (start 140.8435 93.4066) (end 131.0217 93.4066) (width 0.2) (layer "B.Cu") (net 19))
 (segment (start 142.1519 94.715) (end 140.8435 93.4066) (width 0.2) (layer "B.Cu") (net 19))
 (segment (start 161.87 91.93) (end 156.75 97.05) (width 0.2) (layer "B.Cu") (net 19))
 (segment (start 172.84 64.35) (end 185.3 64.35) (width 0.2) (layer "B.Cu") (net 16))
 (segment (start 122.62 77.291) (end 122.62 95.33) (width 0.2) (layer "B.Cu") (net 16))
 (segment (start 122.543951 74.089) (end 121.899 74.733951) (width 0.2) (layer "B.Cu") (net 16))
 (segment (start 185.3 64.35) (end 185.3 51) (width 0.2) (layer "B.Cu") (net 16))
 (segment (start 121.899 76.646049) (end 122.543951 77.291) (width 0.2) (layer "B.Cu") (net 16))
 (segment (start 122.62 53.59) (end 122.62 74.089) (width 0.2) (layer "B.Cu") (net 16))
 (segment (start 125.21 51) (end 122.62 53.59) (width 0.2) (layer "B.Cu") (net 16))
 (segment (start 122.543951 77.291) (end 122.62 77.291) (width 0.2) (layer "B.Cu") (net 16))
 (segment (start 172.84 89.31) (end 172.84 64.35) (width 0.2) (layer "B.Cu") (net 16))
 (segment (start 122.62 95.33) (end 123 95.71) (width 0.2) (layer "B.Cu") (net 16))
 (segment (start 122.62 74.089) (end 122.543951 74.089) (width 0.2) (layer "B.Cu") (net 16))
 (segment (start 121.899 74.733951) (end 121.899 76.646049) (width 0.2) (layer "B.Cu") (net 16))
 (segment (start 185.3 51) (end 125.21 51) (width 0.2) (layer "B.Cu") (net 16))
 (segment (start 176.36 89.31) (end 172.84 89.31) (width 0.2) (layer "B.Cu") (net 16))
 (segment (start 118.16 75.15) (end 117.92 75.39) (width 0.5) (layer "B.Cu") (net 34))
 (segment (start 118.16 55.07) (end 118.16 75.15) (width 0.5) (layer "B.Cu") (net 34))
 (segment (start 113.43 98.84) (end 110.3 95.71) (width 0.2) (layer "B.Cu") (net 12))
 (segment (start 187.24 102.01) (end 187.24 89.93) (width 0.2) (layer "B.Cu") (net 12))
 (segment (start 158.12 116.47) (end 114.33 116.47) (width 0.2) (layer "B.Cu") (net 12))
 (segment (start 114.33 116.47) (end 113.43 115.57) (width 0.2) (layer "B.Cu") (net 12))
 (segment (start 176.36 102.01) (end 187.24 102.01) (width 0.2) (layer "B.Cu") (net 12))
 (segment (start 113.43 111.96) (end 113.43 98.84) (width 0.2) (layer "B.Cu") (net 12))
 (segment (start 113.43 115.57) (end 113.43 111.96) (width 0.2) (layer "B.Cu") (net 12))
 (segment (start 172.58 102.01) (end 158.12 116.47) (width 0.2) (layer "B.Cu") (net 12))
 (segment (start 187.24 89.93) (end 182.26 89.93) (width 0.2) (layer "B.Cu") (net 12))
 (segment (start 176.36 102.01) (end 172.58 102.01) (width 0.2) (layer "B.Cu") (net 12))
 (segment (start 177.12 57.85) (end 180.86 54.11) (width 0.2) (layer "B.Cu") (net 26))
 (segment (start 139.3643 54.78) (end 151.58 54.78) (width 0.2) (layer "B.Cu") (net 26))
 (segment (start 151.58 54.78) (end 154.65 57.85) (width 0.2) (layer "B.Cu") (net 26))
 (segment (start 139.3643 72.6726) (end 139.3643 54.78) (width 0.2) (layer "B.Cu") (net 26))
 (segment (start 154.65 57.85) (end 177.12 57.85) (width 0.2) (layer "B.Cu") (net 26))
 (segment (start 140.78 74.0883) (end 139.3643 72.6726) (width 0.2) (layer "B.Cu") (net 26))
 (segment (start 140.78 75.39) (end 140.78 74.0883) (width 0.2) (layer "B.Cu") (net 26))
 (segment (start 178.71 58.94) (end 180.57 60.8) (width 0.2) (layer "B.Cu") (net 7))
 (segment (start 141.76 55.76) (end 151.21 55.76) (width 0.2) (layer "B.Cu") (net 7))
 (segment (start 141.76 66.7149) (end 141.76 55.76) (width 0.2) (layer "B.Cu") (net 7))
 (segment (start 154.39 58.94) (end 178.71 58.94) (width 0.2) (layer "B.Cu") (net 7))
 (segment (start 138.2649 77.6949) (end 144.4888 77.6949) (width 0.2) (layer "B.Cu") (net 7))
 (segment (start 151.21 55.76) (end 154.39 58.94) (width 0.2) (layer "B.Cu") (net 7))
 (segment (start 138.24 75.39) (end 138.24 77.67) (width 0.2) (layer "B.Cu") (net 7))
 (segment (start 138.24 77.67) (end 138.2649 77.6949) (width 0.2) (layer "B.Cu") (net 7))
 (segment (start 144.4888 77.6949) (end 144.4888 69.4437) (width 0.2) (layer "B.Cu") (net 7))
 (segment (start 144.4888 69.4437) (end 141.76 66.7149) (width 0.2) (layer "B.Cu") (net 7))
 (segment (start 156.04 86.77) (end 125.54 86.77) (width 0.2) (layer "B.Cu") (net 31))
 (segment (start 125.54 86.77) (end 125.54 75.39) (width 0.2) (layer "B.Cu") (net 31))
 (segment (start 148.16 72.8) (end 148.16 58.05) (width 0.2) (layer "B.Cu") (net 22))
 (segment (start 160.8594 90.7406) (end 160.96 90.64) (width 0.2) (layer "B.Cu") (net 22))
 (segment (start 160.96 90.64) (end 160.96 72.8) (width 0.2) (layer "B.Cu") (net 22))
 (segment (start 143.32 93.8083) (end 146.3877 90.7406) (width 0.2) (layer "B.Cu") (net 22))
 (segment (start 160.96 72.8) (end 148.16 72.8) (width 0.2) (layer "B.Cu") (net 22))
 (segment (start 143.32 95.71) (end 143.32 93.8083) (width 0.2) (layer "B.Cu") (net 22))
 (segment (start 146.3877 90.7406) (end 160.8594 90.7406) (width 0.2) (layer "B.Cu") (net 22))
 (segment (start 154.7383 76.61) (end 156.04 76.61) (width 0.2) (layer "B.Cu") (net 27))
 (segment (start 135.7 78.5022) (end 152.8461 78.5022) (width 0.2) (layer "B.Cu") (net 27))
 (segment (start 152.8461 78.5022) (end 154.7383 76.61) (width 0.2) (layer "B.Cu") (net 27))
 (segment (start 135.7 75.39) (end 135.7 78.5022) (width 0.2) (layer "B.Cu") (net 27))
 (segment (start 128.08 75.39) (end 128.08 84.23) (width 0.2) (layer "B.Cu") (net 30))
 (segment (start 128.08 84.23) (end 156.04 84.23) (width 0.2) (layer "B.Cu") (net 30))
 (segment (start 119.6617 113.55) (end 119.6617 111.96) (width 0.2) (layer "B.Cu") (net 10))
 (segment (start 133.16 105.24) (end 124.85 113.55) (width 0.2) (layer "B.Cu") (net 10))
 (segment (start 119.6617 111.96) (end 118.51 111.96) (width 0.2) (layer "B.Cu") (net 10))
 (segment (start 133.16 95.71) (end 133.16 105.24) (width 0.2) (layer "B.Cu") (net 10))
 (segment (start 124.85 113.55) (end 119.6617 113.55) (width 0.2) (layer "B.Cu") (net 10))
 (segment (start 195.81 71.75) (end 185.99 81.57) (width 0.2) (layer "B.Cu") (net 8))
 (segment (start 185.99 81.57) (end 185.99 84.85) (width 0.2) (layer "B.Cu") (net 8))
 (segment (start 185.99 84.85) (end 182.26 84.85) (width 0.2) (layer "B.Cu") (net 8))
 (segment (start 195.81 60.8) (end 195.81 71.75) (width 0.2) (layer "B.Cu") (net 8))
 (segment (start 182.37 77.38) (end 182.38 77.39) (width 0.5) (layer "B.Cu") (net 63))
 (segment (start 179.77 70.62) (end 179.77 87.33) (width 0.2) (layer "B.Cu") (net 54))
 (segment (start 196.1 55.6117) (end 190.9102 60.8015) (width 0.2) (layer "B.Cu") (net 54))
 (segment (start 179.89 87.45) (end 179.95 87.39) (width 0.2) (layer "B.Cu") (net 54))
 (segment (start 190.9102 70.62) (end 179.77 70.62) (width 0.2) (layer "B.Cu") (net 54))
 (segment (start 179.95 87.39) (end 182.26 87.39) (width 0.2) (layer "B.Cu") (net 54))
 (segment (start 196.1 54.11) (end 196.1 55.6117) (width 0.2) (layer "B.Cu") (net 54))
 (segment (start 190.9102 60.8015) (end 190.9102 70.62) (width 0.2) (layer "B.Cu") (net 54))
 (segment (start 179.77 87.33) (end 179.89 87.45) (width 0.2) (layer "B.Cu") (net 54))
 (segment (start 115.62 58.74) (end 115.655 58.775) (width 0.5) (layer "B.Cu") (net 35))
 (segment (start 115.655 58.775) (end 115.655 62.81) (width 0.5) (layer "B.Cu") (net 35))
 (segment (start 115.62 58.74) (end 115.62 55.07) (width 0.5) (layer "B.Cu") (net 35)))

